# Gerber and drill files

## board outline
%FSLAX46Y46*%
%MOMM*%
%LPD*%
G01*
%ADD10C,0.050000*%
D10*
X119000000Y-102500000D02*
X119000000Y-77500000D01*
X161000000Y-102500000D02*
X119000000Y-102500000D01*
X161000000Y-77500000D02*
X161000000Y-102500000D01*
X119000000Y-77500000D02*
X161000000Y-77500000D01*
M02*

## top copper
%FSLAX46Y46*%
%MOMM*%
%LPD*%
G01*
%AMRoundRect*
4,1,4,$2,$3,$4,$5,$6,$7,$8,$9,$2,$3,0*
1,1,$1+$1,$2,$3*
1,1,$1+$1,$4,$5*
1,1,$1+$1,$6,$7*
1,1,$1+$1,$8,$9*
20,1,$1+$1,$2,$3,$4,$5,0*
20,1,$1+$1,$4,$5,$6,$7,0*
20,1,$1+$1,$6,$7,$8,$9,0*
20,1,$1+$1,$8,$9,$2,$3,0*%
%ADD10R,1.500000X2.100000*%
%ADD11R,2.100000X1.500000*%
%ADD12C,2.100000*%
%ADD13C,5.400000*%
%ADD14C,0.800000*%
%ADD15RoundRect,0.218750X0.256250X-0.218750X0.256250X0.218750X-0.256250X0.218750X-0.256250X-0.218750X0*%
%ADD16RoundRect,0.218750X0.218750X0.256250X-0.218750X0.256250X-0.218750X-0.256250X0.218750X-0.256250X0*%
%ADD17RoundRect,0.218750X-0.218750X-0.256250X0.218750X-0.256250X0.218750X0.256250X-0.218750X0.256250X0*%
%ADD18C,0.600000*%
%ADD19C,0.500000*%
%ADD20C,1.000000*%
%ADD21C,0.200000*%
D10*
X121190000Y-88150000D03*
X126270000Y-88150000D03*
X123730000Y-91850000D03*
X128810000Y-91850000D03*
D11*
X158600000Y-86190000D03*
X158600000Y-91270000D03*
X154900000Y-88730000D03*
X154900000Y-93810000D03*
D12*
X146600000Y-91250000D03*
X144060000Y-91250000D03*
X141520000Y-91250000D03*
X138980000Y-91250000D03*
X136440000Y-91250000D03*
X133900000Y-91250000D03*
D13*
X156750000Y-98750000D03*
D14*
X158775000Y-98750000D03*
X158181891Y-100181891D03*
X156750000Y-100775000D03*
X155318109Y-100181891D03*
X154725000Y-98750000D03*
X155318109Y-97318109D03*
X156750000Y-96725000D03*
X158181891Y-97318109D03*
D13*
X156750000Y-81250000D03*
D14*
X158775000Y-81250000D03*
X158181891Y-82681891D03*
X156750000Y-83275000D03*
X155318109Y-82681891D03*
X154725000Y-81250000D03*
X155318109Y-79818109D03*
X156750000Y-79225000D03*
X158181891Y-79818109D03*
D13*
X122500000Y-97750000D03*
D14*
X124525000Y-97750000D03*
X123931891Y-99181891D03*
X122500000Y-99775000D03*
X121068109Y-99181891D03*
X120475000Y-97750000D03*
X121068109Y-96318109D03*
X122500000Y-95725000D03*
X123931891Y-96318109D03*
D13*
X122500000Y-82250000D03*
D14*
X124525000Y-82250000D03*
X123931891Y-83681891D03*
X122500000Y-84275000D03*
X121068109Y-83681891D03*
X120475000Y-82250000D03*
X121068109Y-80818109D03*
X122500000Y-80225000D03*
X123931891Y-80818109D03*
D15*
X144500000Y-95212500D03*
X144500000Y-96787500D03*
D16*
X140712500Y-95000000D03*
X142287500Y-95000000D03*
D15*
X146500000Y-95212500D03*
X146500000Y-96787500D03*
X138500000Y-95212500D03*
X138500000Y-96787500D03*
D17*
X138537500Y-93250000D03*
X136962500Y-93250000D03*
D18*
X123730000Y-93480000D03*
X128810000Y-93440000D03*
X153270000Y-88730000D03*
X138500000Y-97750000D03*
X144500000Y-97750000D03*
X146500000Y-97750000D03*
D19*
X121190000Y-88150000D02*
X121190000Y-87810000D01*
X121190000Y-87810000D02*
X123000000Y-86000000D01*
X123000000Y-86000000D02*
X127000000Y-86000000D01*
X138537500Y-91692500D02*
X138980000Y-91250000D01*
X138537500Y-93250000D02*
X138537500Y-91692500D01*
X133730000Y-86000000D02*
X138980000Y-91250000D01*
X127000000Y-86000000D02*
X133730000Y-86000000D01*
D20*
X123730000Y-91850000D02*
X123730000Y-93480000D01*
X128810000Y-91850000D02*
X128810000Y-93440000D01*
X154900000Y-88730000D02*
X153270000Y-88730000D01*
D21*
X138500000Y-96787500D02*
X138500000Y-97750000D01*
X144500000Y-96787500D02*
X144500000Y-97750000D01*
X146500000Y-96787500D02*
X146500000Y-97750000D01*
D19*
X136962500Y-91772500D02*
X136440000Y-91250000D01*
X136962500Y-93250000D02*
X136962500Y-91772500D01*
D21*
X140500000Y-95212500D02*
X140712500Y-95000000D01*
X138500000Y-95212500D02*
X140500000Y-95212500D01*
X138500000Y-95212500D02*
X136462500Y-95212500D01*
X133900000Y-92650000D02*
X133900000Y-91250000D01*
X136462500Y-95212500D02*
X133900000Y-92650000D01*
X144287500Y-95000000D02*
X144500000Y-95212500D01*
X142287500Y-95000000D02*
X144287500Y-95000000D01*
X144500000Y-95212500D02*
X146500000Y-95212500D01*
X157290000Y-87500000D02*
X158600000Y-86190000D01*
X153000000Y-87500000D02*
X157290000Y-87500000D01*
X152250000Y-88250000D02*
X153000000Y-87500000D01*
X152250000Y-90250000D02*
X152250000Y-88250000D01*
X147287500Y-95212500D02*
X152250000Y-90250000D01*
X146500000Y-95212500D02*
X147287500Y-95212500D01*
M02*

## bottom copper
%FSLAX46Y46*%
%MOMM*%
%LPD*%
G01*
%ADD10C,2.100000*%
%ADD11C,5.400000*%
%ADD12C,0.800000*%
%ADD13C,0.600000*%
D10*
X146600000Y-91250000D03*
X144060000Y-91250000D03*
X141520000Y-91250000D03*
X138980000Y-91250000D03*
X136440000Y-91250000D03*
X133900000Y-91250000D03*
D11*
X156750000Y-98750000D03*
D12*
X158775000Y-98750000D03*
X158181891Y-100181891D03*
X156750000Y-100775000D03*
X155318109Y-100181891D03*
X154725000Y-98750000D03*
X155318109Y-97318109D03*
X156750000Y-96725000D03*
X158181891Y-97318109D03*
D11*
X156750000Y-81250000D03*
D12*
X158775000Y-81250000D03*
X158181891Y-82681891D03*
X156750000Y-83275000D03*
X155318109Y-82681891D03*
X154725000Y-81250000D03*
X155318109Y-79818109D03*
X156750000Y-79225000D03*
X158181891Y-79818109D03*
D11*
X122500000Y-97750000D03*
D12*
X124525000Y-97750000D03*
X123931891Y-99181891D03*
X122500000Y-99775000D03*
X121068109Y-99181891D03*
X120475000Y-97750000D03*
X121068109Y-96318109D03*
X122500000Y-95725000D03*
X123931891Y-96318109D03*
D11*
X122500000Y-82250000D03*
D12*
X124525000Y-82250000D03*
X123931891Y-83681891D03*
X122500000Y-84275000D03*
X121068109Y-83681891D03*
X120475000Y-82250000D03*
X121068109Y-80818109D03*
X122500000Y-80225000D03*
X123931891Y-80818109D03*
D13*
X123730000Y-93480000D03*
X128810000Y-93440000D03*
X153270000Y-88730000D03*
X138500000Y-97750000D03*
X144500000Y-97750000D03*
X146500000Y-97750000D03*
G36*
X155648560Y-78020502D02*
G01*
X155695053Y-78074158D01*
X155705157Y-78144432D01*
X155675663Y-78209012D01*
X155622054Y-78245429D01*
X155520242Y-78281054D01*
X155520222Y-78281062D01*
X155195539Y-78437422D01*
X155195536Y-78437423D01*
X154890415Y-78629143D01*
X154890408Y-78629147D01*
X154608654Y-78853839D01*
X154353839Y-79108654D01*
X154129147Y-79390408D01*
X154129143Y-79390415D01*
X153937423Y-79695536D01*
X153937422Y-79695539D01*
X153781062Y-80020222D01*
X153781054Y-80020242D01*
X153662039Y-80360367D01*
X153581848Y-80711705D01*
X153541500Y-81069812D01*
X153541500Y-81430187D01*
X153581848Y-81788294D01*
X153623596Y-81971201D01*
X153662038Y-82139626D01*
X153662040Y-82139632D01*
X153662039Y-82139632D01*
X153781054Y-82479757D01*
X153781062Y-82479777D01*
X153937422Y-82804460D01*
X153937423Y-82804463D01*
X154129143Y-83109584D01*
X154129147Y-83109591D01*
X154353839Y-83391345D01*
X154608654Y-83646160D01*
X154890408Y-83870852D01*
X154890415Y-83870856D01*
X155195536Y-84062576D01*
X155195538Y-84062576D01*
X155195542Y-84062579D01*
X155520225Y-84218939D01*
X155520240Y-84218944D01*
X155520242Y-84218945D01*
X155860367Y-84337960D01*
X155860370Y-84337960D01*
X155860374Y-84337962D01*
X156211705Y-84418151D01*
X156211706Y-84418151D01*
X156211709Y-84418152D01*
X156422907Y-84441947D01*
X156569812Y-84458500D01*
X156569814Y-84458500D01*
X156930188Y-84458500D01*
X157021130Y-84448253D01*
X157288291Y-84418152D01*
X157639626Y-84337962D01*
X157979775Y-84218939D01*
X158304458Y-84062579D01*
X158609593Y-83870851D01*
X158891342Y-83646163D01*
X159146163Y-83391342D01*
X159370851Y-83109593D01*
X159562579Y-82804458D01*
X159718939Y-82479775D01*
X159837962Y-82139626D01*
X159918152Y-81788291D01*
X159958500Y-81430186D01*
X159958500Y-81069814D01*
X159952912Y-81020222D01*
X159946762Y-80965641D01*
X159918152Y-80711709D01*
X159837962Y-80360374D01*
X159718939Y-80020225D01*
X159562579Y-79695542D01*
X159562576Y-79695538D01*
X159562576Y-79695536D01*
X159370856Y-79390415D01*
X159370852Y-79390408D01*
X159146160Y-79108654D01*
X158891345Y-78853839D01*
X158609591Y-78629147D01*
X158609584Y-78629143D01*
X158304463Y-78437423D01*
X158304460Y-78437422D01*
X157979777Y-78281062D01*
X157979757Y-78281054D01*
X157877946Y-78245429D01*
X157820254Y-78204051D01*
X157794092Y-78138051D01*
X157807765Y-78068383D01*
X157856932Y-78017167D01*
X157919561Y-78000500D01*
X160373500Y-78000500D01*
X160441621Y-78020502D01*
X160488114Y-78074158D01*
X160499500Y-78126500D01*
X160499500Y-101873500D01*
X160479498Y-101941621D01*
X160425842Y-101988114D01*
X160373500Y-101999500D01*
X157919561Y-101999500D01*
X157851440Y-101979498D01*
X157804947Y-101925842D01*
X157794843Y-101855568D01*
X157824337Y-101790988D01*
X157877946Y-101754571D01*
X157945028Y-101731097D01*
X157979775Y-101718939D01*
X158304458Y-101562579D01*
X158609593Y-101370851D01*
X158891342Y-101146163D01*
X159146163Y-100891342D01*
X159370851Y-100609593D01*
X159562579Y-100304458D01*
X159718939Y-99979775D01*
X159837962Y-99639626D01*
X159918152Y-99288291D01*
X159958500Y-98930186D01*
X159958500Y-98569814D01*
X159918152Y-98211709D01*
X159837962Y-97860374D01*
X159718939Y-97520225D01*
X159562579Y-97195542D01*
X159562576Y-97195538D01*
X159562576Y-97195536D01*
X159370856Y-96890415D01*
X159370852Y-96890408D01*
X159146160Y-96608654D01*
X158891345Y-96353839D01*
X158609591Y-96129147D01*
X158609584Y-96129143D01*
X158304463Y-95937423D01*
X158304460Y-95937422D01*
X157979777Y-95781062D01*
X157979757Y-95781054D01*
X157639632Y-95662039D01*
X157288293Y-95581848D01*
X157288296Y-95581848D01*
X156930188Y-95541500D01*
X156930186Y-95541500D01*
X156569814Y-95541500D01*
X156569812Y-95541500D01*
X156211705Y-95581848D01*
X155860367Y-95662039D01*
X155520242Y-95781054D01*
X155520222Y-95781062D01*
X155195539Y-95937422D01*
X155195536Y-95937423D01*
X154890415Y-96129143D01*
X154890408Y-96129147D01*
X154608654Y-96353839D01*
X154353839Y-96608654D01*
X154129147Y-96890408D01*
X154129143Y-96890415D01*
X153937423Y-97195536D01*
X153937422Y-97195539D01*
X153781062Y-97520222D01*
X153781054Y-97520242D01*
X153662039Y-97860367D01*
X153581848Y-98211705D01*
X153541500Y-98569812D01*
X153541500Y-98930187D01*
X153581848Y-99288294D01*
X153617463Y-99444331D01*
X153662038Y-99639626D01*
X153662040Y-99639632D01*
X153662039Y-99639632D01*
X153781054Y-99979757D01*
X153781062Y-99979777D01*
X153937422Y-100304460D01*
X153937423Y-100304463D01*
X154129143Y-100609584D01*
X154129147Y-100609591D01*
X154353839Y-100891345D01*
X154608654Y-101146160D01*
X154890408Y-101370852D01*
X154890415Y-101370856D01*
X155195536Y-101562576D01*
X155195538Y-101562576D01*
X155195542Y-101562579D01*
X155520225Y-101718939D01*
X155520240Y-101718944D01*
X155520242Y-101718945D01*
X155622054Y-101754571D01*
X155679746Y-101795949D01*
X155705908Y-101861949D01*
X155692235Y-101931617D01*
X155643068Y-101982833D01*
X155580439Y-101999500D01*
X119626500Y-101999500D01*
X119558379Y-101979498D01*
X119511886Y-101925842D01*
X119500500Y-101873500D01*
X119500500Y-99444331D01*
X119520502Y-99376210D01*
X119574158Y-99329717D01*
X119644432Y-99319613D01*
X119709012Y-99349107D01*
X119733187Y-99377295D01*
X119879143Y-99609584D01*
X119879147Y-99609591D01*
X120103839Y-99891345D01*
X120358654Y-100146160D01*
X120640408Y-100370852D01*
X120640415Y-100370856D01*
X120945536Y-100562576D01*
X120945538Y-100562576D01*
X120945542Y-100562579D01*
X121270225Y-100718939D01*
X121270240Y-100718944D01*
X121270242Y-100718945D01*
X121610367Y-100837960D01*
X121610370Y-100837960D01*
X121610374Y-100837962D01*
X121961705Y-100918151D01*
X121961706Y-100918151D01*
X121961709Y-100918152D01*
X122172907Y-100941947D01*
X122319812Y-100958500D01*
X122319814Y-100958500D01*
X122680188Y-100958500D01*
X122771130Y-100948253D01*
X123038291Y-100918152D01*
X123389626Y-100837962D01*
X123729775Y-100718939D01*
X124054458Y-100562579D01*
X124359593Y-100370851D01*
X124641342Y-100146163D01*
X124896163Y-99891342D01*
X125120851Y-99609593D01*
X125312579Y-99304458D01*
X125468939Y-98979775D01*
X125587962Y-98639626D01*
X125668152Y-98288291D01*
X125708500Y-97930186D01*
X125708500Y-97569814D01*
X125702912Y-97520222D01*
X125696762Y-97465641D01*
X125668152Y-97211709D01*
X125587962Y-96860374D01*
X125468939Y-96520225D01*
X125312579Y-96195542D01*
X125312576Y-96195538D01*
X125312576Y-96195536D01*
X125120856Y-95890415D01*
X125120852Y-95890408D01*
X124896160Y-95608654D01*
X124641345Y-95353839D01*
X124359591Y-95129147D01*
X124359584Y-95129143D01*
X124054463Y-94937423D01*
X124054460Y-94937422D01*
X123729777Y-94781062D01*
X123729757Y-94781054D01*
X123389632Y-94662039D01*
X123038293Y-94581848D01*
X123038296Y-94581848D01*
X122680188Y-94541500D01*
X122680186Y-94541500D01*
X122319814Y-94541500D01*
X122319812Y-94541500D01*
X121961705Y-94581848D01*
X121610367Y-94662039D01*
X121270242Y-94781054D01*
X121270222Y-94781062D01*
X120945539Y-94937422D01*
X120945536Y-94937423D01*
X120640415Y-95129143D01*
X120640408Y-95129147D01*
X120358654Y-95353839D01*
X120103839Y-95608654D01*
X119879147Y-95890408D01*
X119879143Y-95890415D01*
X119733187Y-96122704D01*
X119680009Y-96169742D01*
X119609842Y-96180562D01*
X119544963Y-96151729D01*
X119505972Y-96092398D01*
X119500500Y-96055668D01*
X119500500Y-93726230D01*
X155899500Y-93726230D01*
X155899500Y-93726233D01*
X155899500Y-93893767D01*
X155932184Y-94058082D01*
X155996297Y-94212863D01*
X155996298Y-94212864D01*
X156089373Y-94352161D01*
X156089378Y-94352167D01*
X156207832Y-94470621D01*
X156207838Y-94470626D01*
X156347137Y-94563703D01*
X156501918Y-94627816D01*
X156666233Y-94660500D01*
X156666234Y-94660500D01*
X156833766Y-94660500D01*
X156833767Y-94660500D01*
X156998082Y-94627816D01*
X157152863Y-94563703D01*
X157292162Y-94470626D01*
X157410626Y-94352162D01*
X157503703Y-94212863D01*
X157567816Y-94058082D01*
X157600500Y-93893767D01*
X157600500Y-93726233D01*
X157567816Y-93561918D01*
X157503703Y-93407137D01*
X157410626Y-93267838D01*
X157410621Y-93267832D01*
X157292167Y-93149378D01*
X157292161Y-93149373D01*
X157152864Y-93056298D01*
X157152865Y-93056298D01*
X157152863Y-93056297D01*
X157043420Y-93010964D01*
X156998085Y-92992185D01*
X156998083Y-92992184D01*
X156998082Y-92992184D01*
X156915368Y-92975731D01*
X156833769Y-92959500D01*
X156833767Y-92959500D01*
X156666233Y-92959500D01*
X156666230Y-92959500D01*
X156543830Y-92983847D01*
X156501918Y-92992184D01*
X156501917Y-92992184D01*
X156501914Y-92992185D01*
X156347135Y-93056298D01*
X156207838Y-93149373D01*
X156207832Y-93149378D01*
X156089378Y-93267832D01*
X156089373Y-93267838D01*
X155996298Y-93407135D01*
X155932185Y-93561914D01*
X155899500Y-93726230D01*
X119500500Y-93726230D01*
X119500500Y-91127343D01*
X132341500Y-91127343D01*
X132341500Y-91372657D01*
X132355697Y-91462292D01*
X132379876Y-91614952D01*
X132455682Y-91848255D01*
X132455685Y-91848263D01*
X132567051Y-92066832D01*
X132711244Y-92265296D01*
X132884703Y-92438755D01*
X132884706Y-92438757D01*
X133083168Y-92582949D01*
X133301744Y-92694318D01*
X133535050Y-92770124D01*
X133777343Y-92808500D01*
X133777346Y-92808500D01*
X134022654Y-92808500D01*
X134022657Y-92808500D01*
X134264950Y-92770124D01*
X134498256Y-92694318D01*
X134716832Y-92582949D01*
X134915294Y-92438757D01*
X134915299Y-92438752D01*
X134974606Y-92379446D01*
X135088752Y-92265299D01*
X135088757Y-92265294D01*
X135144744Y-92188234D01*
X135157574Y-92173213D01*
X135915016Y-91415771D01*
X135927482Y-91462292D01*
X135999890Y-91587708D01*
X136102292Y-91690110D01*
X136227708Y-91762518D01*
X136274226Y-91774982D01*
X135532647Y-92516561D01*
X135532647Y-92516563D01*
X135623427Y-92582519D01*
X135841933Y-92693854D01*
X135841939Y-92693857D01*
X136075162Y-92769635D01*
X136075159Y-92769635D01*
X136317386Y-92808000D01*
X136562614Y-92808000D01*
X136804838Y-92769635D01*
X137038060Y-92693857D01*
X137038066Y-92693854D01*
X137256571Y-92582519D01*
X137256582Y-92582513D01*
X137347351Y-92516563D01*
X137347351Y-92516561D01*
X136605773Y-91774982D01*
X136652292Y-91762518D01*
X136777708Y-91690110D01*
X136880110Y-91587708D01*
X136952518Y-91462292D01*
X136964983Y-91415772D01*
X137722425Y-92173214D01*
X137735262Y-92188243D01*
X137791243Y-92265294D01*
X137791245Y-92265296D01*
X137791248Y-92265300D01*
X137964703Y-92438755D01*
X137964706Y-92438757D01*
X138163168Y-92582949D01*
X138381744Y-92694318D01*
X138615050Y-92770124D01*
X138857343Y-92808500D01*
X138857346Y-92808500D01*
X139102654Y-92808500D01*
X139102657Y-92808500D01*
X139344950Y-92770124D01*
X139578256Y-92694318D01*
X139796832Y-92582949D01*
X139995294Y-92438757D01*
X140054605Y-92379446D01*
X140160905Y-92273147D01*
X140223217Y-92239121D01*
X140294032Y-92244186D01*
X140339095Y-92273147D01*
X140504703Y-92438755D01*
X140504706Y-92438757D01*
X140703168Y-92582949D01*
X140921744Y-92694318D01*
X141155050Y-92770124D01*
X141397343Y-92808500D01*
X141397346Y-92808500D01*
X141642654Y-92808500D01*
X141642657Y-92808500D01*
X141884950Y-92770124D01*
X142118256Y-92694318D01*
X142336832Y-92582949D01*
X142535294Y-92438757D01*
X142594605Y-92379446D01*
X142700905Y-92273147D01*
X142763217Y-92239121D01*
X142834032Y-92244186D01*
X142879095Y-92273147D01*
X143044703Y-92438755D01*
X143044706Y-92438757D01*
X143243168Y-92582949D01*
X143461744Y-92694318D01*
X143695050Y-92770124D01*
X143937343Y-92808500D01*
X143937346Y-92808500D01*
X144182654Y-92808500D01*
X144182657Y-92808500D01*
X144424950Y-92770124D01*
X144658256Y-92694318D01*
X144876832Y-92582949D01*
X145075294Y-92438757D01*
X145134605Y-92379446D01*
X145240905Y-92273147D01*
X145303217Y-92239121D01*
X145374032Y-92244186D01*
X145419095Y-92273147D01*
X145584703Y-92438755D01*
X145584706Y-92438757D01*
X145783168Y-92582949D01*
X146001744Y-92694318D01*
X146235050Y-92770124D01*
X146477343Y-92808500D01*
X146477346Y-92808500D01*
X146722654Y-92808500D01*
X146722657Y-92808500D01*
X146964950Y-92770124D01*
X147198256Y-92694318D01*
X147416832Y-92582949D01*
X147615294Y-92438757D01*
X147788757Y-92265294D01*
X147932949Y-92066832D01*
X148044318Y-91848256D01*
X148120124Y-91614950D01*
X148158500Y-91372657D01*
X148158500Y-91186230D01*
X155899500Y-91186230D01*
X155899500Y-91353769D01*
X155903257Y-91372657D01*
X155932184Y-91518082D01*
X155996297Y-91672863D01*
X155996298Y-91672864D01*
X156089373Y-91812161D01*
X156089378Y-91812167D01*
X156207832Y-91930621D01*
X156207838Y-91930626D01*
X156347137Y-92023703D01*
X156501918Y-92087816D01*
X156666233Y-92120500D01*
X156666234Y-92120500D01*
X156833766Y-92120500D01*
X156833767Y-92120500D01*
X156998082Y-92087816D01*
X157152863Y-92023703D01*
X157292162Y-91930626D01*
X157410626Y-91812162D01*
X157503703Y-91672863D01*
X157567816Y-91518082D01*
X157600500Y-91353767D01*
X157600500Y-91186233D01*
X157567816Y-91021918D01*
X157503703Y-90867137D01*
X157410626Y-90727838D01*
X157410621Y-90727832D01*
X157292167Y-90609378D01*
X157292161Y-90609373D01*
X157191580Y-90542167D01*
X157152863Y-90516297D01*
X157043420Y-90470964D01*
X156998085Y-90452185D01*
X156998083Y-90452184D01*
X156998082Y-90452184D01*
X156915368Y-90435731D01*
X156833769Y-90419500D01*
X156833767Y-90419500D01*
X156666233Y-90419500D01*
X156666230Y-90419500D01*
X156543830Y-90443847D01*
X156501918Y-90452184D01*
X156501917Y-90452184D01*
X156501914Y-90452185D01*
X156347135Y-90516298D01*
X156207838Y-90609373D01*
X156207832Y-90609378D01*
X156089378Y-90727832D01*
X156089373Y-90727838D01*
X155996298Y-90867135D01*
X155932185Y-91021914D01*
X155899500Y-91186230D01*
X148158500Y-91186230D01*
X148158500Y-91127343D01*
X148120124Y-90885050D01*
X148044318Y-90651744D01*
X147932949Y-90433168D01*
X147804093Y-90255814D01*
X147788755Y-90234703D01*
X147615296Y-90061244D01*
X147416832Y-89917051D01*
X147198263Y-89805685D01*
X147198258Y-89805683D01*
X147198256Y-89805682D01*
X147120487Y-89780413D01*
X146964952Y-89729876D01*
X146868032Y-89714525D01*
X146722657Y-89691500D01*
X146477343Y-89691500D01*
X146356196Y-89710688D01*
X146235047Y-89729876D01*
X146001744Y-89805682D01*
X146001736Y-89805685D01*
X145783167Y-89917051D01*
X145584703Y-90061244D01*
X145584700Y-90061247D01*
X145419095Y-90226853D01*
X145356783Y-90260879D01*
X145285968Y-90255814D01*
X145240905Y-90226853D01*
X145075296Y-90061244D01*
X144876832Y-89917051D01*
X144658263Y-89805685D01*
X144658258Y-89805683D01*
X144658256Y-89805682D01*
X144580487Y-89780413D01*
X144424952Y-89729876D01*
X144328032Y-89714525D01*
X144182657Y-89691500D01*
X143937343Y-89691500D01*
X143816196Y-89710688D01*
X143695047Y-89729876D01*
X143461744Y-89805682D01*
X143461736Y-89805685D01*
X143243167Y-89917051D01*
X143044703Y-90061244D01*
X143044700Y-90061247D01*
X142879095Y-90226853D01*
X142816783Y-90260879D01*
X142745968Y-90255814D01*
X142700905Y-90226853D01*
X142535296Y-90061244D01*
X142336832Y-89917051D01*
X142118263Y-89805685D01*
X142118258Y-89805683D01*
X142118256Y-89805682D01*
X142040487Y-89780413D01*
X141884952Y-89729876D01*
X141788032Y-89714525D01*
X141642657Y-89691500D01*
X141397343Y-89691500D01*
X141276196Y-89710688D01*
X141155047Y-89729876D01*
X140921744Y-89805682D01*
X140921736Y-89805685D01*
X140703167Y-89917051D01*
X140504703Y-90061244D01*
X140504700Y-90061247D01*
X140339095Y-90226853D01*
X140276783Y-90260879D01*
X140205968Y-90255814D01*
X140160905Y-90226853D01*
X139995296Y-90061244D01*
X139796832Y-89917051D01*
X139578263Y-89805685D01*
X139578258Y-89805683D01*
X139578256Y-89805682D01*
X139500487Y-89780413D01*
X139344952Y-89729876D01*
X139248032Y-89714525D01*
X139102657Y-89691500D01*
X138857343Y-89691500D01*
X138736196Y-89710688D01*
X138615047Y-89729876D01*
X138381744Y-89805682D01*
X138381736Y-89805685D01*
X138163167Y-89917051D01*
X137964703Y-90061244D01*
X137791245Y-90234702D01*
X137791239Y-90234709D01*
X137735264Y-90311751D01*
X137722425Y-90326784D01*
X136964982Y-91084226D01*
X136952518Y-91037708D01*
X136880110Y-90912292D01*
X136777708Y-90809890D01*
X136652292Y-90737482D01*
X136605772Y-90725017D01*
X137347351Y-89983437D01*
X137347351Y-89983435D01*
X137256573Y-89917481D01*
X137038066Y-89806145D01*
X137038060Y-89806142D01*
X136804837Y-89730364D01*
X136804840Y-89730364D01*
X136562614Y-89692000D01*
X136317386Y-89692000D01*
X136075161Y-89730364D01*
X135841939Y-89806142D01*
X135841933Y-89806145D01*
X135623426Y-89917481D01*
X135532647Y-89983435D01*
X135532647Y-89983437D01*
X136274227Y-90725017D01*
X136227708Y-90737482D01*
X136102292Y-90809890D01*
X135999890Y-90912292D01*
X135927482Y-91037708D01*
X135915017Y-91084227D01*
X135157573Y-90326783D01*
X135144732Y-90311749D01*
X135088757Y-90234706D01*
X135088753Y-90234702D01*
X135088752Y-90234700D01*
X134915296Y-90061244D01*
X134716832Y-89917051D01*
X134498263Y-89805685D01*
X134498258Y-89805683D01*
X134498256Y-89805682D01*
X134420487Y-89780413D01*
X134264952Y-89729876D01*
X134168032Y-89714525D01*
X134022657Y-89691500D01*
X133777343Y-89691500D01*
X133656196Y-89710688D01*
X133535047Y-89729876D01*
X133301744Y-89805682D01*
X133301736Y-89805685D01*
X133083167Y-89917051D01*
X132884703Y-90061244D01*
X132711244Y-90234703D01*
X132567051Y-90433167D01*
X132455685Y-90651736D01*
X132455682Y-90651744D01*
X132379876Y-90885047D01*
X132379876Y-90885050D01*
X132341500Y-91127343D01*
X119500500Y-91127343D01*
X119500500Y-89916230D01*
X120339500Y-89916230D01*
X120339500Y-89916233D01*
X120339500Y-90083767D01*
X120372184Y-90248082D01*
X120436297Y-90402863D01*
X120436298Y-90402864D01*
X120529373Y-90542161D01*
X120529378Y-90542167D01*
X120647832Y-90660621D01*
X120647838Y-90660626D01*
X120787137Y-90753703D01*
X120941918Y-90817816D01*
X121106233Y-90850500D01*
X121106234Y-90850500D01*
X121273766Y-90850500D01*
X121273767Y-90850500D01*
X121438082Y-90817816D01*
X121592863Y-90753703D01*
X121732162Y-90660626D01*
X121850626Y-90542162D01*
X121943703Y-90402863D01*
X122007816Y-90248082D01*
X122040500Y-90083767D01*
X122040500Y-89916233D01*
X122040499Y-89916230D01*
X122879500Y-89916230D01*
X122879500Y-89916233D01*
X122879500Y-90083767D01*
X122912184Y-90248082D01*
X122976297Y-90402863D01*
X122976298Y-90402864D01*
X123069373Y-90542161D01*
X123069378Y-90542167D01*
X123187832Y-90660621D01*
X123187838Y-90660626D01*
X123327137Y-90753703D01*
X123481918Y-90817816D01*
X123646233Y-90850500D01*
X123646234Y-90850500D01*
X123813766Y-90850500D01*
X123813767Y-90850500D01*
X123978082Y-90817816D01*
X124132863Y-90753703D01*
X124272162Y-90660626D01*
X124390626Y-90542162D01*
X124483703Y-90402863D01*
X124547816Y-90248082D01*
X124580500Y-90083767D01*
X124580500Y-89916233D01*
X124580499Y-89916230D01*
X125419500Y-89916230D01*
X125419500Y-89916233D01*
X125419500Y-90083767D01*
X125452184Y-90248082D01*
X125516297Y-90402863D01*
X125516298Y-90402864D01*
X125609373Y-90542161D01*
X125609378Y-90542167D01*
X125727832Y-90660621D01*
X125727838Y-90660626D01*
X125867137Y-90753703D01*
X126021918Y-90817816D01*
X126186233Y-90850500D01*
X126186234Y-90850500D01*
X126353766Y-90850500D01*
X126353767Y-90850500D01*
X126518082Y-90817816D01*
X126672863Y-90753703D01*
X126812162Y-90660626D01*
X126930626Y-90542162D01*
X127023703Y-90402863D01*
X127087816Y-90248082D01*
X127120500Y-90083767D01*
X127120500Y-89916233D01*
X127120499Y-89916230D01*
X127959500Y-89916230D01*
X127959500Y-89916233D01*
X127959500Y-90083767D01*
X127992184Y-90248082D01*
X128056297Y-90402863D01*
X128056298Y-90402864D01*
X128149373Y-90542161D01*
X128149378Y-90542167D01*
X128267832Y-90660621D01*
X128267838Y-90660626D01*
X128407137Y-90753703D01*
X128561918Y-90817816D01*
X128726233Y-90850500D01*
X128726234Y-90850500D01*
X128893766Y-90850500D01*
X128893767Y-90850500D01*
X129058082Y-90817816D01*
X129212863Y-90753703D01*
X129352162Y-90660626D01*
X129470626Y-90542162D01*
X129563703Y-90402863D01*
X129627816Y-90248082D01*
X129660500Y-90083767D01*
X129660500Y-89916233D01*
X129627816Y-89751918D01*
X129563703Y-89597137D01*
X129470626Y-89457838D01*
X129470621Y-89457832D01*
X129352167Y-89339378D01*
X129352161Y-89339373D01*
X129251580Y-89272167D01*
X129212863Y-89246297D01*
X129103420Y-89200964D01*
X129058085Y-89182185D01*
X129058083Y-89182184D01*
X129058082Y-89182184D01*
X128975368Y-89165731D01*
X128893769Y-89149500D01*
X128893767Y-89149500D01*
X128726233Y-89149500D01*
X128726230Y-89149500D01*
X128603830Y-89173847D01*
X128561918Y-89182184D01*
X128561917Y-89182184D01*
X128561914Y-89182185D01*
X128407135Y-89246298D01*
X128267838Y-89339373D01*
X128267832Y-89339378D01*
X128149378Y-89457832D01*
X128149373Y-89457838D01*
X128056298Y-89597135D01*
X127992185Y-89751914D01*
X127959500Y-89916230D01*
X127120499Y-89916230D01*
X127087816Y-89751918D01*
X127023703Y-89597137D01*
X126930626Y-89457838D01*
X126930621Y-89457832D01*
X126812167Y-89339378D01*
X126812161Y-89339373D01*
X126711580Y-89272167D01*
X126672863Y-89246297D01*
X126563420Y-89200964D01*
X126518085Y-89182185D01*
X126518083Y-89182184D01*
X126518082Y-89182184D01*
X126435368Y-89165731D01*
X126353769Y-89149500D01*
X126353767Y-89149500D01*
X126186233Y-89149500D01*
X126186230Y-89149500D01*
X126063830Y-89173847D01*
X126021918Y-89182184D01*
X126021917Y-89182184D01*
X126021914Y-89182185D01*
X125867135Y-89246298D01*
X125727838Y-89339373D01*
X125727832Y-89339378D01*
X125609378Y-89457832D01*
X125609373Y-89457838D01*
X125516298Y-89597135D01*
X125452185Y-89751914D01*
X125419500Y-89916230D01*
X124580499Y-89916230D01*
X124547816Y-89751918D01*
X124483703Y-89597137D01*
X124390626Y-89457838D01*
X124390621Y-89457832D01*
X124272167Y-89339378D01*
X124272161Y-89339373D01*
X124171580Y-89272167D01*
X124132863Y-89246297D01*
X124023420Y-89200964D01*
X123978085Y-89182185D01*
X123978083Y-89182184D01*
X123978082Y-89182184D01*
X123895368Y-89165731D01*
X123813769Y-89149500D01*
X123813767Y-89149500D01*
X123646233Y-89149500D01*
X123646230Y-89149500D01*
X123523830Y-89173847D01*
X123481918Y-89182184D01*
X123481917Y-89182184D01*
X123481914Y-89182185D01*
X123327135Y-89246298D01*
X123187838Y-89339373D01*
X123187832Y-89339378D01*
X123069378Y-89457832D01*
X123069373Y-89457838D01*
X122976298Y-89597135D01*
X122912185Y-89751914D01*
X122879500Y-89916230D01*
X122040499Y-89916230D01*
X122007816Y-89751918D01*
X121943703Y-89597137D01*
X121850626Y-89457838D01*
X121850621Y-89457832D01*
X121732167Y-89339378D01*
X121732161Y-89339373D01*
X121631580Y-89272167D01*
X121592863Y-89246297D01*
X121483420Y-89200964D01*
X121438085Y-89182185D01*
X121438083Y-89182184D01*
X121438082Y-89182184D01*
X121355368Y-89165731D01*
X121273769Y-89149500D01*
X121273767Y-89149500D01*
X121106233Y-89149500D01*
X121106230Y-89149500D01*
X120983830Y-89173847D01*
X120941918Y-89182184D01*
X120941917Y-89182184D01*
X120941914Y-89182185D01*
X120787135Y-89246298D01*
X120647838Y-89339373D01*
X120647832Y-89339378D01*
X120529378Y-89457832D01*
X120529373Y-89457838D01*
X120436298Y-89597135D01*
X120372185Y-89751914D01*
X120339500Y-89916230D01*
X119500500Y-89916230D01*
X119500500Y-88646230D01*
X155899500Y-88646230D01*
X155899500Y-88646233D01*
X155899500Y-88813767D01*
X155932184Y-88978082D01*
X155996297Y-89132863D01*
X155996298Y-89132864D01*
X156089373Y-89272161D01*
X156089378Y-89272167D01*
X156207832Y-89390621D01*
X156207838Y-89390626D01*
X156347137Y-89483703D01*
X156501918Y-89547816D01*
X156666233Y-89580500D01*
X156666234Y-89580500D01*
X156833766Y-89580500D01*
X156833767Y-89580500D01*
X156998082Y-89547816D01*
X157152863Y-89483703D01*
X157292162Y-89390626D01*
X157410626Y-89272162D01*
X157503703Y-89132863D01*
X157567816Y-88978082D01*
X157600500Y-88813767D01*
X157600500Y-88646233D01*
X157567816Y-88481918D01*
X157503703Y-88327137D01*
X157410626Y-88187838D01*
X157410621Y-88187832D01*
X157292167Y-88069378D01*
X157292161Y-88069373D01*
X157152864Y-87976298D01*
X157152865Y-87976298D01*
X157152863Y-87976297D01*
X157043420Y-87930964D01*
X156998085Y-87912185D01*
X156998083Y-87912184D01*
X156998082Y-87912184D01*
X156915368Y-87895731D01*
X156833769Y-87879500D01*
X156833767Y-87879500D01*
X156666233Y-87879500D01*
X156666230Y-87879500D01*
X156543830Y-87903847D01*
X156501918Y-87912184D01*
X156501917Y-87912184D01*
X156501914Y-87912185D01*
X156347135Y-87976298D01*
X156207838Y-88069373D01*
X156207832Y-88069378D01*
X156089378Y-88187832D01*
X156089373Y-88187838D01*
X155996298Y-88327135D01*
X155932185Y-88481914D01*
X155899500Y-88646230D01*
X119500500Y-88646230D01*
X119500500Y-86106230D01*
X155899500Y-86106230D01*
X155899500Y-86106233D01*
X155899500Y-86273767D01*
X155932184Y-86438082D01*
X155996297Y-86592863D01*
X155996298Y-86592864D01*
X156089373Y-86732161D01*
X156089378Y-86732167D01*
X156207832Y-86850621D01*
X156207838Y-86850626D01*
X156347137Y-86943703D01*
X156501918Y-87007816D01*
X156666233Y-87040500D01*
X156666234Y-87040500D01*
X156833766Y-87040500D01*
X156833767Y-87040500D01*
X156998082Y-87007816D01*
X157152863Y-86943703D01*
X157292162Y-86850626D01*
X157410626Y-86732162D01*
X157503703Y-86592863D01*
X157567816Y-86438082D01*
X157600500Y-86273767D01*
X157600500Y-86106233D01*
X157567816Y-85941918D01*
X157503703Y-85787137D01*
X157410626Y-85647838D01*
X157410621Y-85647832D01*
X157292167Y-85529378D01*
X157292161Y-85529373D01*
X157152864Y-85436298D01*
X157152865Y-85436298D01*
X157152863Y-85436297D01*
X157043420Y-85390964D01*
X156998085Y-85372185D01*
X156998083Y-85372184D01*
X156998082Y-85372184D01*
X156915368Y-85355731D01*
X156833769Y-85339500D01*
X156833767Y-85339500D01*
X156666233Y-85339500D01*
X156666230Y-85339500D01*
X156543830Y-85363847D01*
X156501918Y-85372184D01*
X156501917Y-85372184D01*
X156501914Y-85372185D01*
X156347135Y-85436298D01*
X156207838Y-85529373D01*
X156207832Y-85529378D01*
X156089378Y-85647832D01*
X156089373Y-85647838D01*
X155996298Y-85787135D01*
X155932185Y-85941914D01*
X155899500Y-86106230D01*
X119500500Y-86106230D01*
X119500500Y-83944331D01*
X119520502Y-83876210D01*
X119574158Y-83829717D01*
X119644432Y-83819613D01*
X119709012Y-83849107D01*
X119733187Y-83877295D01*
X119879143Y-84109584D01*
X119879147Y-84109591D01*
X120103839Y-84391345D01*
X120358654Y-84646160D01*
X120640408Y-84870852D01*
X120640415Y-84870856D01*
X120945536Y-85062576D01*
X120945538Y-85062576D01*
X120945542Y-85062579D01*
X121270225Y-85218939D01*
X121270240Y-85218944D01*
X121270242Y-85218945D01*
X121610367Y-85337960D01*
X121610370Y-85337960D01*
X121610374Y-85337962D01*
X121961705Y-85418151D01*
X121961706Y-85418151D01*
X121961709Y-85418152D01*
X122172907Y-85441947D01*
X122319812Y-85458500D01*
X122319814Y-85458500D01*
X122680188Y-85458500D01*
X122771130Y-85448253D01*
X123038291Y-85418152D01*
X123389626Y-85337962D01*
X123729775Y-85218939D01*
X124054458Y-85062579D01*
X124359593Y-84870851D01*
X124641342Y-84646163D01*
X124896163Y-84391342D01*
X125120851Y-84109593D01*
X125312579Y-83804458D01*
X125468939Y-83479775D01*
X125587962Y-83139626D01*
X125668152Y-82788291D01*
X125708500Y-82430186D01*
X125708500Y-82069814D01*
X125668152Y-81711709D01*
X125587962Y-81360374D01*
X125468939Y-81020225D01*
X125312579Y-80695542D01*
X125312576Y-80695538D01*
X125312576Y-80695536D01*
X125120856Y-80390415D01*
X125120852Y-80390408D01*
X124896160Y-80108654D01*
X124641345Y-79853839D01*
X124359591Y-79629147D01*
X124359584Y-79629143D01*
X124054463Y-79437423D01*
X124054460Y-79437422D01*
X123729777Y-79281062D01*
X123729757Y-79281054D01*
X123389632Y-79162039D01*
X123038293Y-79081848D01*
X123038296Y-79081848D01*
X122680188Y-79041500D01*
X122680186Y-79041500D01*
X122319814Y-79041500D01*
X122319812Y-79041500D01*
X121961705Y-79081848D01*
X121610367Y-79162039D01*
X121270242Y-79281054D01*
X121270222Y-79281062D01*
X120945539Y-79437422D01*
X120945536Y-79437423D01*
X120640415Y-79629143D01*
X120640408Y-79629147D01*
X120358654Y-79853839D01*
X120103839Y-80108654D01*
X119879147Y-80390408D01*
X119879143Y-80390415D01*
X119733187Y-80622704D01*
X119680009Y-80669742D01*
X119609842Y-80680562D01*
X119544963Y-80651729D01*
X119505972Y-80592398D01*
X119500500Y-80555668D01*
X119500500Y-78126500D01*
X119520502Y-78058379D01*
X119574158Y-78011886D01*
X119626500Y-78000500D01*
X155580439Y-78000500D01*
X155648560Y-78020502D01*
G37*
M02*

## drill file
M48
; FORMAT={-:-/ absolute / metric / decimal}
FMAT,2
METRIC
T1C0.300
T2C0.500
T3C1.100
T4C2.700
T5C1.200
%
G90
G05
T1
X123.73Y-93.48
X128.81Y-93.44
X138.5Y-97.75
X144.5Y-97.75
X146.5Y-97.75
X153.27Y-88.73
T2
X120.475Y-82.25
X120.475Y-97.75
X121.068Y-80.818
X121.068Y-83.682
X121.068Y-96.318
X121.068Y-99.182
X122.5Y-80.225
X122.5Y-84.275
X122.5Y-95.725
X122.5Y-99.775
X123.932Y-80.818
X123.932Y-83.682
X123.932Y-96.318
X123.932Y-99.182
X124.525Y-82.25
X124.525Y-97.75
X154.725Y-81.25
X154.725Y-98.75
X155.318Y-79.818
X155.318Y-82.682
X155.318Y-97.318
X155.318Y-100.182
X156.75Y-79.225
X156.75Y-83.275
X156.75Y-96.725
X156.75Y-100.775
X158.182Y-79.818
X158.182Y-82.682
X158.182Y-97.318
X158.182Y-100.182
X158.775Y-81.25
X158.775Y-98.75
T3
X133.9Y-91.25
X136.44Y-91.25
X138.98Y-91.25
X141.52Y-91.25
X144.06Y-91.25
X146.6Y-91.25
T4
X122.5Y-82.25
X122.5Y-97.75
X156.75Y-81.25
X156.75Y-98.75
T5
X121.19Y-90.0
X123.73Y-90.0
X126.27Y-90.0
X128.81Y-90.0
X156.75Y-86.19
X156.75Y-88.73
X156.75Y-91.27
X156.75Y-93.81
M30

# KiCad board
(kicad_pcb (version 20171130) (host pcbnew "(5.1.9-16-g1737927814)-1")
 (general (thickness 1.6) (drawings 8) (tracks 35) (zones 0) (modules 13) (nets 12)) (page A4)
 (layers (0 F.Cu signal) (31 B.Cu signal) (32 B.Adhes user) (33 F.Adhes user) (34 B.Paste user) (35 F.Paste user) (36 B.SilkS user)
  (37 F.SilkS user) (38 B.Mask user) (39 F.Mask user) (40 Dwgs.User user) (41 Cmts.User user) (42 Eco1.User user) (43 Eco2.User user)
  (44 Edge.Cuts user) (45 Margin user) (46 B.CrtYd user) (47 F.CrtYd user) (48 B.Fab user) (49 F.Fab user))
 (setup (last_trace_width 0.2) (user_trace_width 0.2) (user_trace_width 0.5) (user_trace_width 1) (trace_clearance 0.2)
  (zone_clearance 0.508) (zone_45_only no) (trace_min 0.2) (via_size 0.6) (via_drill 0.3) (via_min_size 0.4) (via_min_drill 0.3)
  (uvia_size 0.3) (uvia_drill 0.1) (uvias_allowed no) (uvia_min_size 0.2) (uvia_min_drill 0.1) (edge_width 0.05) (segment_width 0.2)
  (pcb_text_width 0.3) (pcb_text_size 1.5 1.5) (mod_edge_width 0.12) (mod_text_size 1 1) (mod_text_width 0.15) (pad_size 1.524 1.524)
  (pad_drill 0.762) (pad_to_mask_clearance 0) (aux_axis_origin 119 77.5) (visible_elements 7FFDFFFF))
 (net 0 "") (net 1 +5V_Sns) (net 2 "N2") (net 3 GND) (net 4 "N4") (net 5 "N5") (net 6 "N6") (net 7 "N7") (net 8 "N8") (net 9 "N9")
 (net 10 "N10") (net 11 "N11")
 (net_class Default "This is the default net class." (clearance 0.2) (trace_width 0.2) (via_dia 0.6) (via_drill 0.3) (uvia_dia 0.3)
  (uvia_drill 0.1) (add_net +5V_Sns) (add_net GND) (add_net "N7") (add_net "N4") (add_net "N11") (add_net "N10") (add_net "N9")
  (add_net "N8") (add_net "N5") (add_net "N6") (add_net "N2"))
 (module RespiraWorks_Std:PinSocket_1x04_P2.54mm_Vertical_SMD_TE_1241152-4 (layer F.Cu) (at 125 90 90)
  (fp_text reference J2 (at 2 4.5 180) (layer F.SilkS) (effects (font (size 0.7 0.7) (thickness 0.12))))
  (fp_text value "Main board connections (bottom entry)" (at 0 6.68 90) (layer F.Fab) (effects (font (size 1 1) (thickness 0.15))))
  (pad "" np_thru_hole circle (at 0 1.27 90) (size 1.2 1.2) (drill 1.2) (layers *.Cu *.Mask))
  (pad "" np_thru_hole circle (at 0 -1.27 90) (size 1.2 1.2) (drill 1.2) (layers *.Cu *.Mask))
  (pad "" np_thru_hole circle (at 0 -3.81 90) (size 1.2 1.2) (drill 1.2) (layers *.Cu *.Mask))
  (pad 1 smd rect (at 1.85 -3.81 90) (size 2.1 1.5) (layers F.Cu F.Paste F.Mask) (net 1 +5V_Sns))
  (pad 3 smd rect (at 1.85 1.27 90) (size 2.1 1.5) (layers F.Cu F.Paste F.Mask) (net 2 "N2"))
  (pad 2 smd rect (at -1.85 -1.27 90) (size 2.1 1.5) (layers F.Cu F.Paste F.Mask) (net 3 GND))
  (pad 4 smd rect (at -1.85 3.81 90) (size 2.1 1.5) (layers F.Cu F.Paste F.Mask) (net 3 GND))
  (pad "" np_thru_hole circle (at 0 3.81 90) (size 1.2 1.2) (drill 1.2) (layers *.Cu *.Mask)))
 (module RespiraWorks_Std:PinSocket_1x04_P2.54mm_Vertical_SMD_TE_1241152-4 (layer F.Cu) (at 156.75 90)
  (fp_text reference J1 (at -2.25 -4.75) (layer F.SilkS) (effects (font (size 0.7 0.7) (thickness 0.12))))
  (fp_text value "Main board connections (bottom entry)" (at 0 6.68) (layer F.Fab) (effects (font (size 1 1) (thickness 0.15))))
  (pad "" np_thru_hole circle (at 0 1.27) (size 1.2 1.2) (drill 1.2) (layers *.Cu *.Mask))
  (pad "" np_thru_hole circle (at 0 -1.27) (size 1.2 1.2) (drill 1.2) (layers *.Cu *.Mask))
  (pad "" np_thru_hole circle (at 0 -3.81) (size 1.2 1.2) (drill 1.2) (layers *.Cu *.Mask))
  (pad 1 smd rect (at 1.85 -3.81) (size 2.1 1.5) (layers F.Cu F.Paste F.Mask) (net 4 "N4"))
  (pad 3 smd rect (at 1.85 1.27) (size 2.1 1.5) (layers F.Cu F.Paste F.Mask) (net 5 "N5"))
  (pad 2 smd rect (at -1.85 -1.27) (size 2.1 1.5) (layers F.Cu F.Paste F.Mask) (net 3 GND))
  (pad 4 smd rect (at -1.85 3.81) (size 2.1 1.5) (layers F.Cu F.Paste F.Mask) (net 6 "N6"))
  (pad "" np_thru_hole circle (at 0 3.81) (size 1.2 1.2) (drill 1.2) (layers *.Cu *.Mask)))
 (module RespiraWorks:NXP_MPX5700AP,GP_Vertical (layer F.Cu) (at 140.25 91.25)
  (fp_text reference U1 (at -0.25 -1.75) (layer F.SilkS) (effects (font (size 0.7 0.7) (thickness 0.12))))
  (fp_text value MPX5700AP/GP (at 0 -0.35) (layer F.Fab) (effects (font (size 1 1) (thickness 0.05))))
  (pad 6 thru_hole circle (at 6.35 0) (size 2.1 2.1) (drill 1.1) (layers *.Cu *.Mask))
  (pad 5 thru_hole circle (at 3.81 0) (size 2.1 2.1) (drill 1.1) (layers *.Cu *.Mask))
  (pad 4 thru_hole circle (at 1.27 0) (size 2.1 2.1) (drill 1.1) (layers *.Cu *.Mask))
  (pad 3 thru_hole circle (at -1.27 0) (size 2.1 2.1) (drill 1.1) (layers *.Cu *.Mask) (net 1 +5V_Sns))
  (pad 2 thru_hole circle (at -3.81 0) (size 2.1 2.1) (drill 1.1) (layers *.Cu *.Mask) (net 3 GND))
  (pad 1 thru_hole circle (at -6.35 0) (size 2.1 2.1) (drill 1.1) (layers *.Cu *.Mask) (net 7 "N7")))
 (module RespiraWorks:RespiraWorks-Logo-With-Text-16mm (layer B.Cu) (at 139.5 89.75 180)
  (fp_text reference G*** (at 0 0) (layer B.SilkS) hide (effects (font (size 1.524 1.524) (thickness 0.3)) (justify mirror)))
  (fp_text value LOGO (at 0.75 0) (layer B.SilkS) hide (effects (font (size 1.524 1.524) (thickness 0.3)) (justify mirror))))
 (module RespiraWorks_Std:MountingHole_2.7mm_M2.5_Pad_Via (layer F.Cu) (at 156.75 98.75)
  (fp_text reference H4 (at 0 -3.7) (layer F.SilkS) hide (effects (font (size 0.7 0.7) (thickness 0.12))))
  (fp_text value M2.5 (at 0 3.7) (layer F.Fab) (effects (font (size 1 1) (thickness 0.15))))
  (pad 1 thru_hole circle (at 0 0) (size 5.4 5.4) (drill 2.7) (layers *.Cu *.Mask) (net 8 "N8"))
  (pad 1 thru_hole circle (at 2.025 0) (size 0.8 0.8) (drill 0.5) (layers *.Cu *.Mask) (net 8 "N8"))
  (pad 1 thru_hole circle (at 1.431891 1.431891) (size 0.8 0.8) (drill 0.5) (layers *.Cu *.Mask) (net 8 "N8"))
  (pad 1 thru_hole circle (at 0 2.025) (size 0.8 0.8) (drill 0.5) (layers *.Cu *.Mask) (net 8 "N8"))
  (pad 1 thru_hole circle (at -1.431891 1.431891) (size 0.8 0.8) (drill 0.5) (layers *.Cu *.Mask) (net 8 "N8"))
  (pad 1 thru_hole circle (at -2.025 0) (size 0.8 0.8) (drill 0.5) (layers *.Cu *.Mask) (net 8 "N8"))
  (pad 1 thru_hole circle (at -1.431891 -1.431891) (size 0.8 0.8) (drill 0.5) (layers *.Cu *.Mask) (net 8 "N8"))
  (pad 1 thru_hole circle (at 0 -2.025) (size 0.8 0.8) (drill 0.5) (layers *.Cu *.Mask) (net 8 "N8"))
  (pad 1 thru_hole circle (at 1.431891 -1.431891) (size 0.8 0.8) (drill 0.5) (layers *.Cu *.Mask) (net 8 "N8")))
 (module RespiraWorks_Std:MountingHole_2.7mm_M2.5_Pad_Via (layer F.Cu) (at 156.75 81.25)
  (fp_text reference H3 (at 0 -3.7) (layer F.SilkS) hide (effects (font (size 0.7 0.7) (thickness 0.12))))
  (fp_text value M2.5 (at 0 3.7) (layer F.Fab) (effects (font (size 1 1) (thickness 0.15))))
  (pad 1 thru_hole circle (at 0 0) (size 5.4 5.4) (drill 2.7) (layers *.Cu *.Mask) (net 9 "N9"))
  (pad 1 thru_hole circle (at 2.025 0) (size 0.8 0.8) (drill 0.5) (layers *.Cu *.Mask) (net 9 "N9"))
  (pad 1 thru_hole circle (at 1.431891 1.431891) (size 0.8 0.8) (drill 0.5) (layers *.Cu *.Mask) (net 9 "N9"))
  (pad 1 thru_hole circle (at 0 2.025) (size 0.8 0.8) (drill 0.5) (layers *.Cu *.Mask) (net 9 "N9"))
  (pad 1 thru_hole circle (at -1.431891 1.431891) (size 0.8 0.8) (drill 0.5) (layers *.Cu *.Mask) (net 9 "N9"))
  (pad 1 thru_hole circle (at -2.025 0) (size 0.8 0.8) (drill 0.5) (layers *.Cu *.Mask) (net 9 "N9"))
  (pad 1 thru_hole circle (at -1.431891 -1.431891) (size 0.8 0.8) (drill 0.5) (layers *.Cu *.Mask) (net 9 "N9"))
  (pad 1 thru_hole circle (at 0 -2.025) (size 0.8 0.8) (drill 0.5) (layers *.Cu *.Mask) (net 9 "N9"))
  (pad 1 thru_hole circle (at 1.431891 -1.431891) (size 0.8 0.8) (drill 0.5) (layers *.Cu *.Mask) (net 9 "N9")))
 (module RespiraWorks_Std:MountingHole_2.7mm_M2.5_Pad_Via (layer F.Cu) (at 122.5 97.75)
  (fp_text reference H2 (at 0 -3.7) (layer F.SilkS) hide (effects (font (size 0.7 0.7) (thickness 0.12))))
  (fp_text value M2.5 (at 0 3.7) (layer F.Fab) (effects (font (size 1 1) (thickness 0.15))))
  (pad 1 thru_hole circle (at 0 0) (size 5.4 5.4) (drill 2.7) (layers *.Cu *.Mask) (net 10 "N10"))
  (pad 1 thru_hole circle (at 2.025 0) (size 0.8 0.8) (drill 0.5) (layers *.Cu *.Mask) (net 10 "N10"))
  (pad 1 thru_hole circle (at 1.431891 1.431891) (size 0.8 0.8) (drill 0.5) (layers *.Cu *.Mask) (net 10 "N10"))
  (pad 1 thru_hole circle (at 0 2.025) (size 0.8 0.8) (drill 0.5) (layers *.Cu *.Mask) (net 10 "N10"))
  (pad 1 thru_hole circle (at -1.431891 1.431891) (size 0.8 0.8) (drill 0.5) (layers *.Cu *.Mask) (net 10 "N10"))
  (pad 1 thru_hole circle (at -2.025 0) (size 0.8 0.8) (drill 0.5) (layers *.Cu *.Mask) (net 10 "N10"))
  (pad 1 thru_hole circle (at -1.431891 -1.431891) (size 0.8 0.8) (drill 0.5) (layers *.Cu *.Mask) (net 10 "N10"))
  (pad 1 thru_hole circle (at 0 -2.025) (size 0.8 0.8) (drill 0.5) (layers *.Cu *.Mask) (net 10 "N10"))
  (pad 1 thru_hole circle (at 1.431891 -1.431891) (size 0.8 0.8) (drill 0.5) (layers *.Cu *.Mask) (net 10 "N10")))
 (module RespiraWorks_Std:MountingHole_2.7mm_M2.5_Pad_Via (layer F.Cu) (at 122.5 82.25)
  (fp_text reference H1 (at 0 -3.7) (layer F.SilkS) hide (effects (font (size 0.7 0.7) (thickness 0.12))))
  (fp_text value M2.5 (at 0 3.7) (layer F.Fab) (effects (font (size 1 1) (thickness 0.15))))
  (pad 1 thru_hole circle (at 0 0) (size 5.4 5.4) (drill 2.7) (layers *.Cu *.Mask) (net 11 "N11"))
  (pad 1 thru_hole circle (at 2.025 0) (size 0.8 0.8) (drill 0.5) (layers *.Cu *.Mask) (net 11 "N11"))
  (pad 1 thru_hole circle (at 1.431891 1.431891) (size 0.8 0.8) (drill 0.5) (layers *.Cu *.Mask) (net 11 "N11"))
  (pad 1 thru_hole circle (at 0 2.025) (size 0.8 0.8) (drill 0.5) (layers *.Cu *.Mask) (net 11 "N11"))
  (pad 1 thru_hole circle (at -1.431891 1.431891) (size 0.8 0.8) (drill 0.5) (layers *.Cu *.Mask) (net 11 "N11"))
  (pad 1 thru_hole circle (at -2.025 0) (size 0.8 0.8) (drill 0.5) (layers *.Cu *.Mask) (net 11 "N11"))
  (pad 1 thru_hole circle (at -1.431891 -1.431891) (size 0.8 0.8) (drill 0.5) (layers *.Cu *.Mask) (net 11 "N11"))
  (pad 1 thru_hole circle (at 0 -2.025) (size 0.8 0.8) (drill 0.5) (layers *.Cu *.Mask) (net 11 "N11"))
  (pad 1 thru_hole circle (at 1.431891 -1.431891) (size 0.8 0.8) (drill 0.5) (layers *.Cu *.Mask) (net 11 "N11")))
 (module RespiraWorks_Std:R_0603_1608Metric (layer F.Cu) (at 144.5 96 90)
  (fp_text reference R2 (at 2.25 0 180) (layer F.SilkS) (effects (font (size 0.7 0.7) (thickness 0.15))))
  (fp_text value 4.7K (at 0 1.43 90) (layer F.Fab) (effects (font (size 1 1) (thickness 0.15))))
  (pad 2 smd roundrect (at 0.7875 0 90) (size 0.875 0.95) (layers F.Cu F.Paste F.Mask) (roundrect_rratio 0.25) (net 4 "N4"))
  (pad 1 smd roundrect (at -0.7875 0 90) (size 0.875 0.95) (layers F.Cu F.Paste F.Mask) (roundrect_rratio 0.25) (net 3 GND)))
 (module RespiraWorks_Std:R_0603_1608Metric (layer F.Cu) (at 141.5 95 180)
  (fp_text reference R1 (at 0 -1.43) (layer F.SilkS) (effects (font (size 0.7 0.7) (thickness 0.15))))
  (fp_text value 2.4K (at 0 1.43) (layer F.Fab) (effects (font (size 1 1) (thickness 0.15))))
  (pad 2 smd roundrect (at 0.7875 0 180) (size 0.875 0.95) (layers F.Cu F.Paste F.Mask) (roundrect_rratio 0.25) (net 7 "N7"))
  (pad 1 smd roundrect (at -0.7875 0 180) (size 0.875 0.95) (layers F.Cu F.Paste F.Mask) (roundrect_rratio 0.25) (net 4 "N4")))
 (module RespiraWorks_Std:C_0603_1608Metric (layer F.Cu) (at 146.5 96 90)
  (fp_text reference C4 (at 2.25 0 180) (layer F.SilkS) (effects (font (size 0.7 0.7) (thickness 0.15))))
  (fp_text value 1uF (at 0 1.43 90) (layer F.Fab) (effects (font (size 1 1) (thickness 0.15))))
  (pad 2 smd roundrect (at 0.7875 0 90) (size 0.875 0.95) (layers F.Cu F.Paste F.Mask) (roundrect_rratio 0.25) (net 4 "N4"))
  (pad 1 smd roundrect (at -0.7875 0 90) (size 0.875 0.95) (layers F.Cu F.Paste F.Mask) (roundrect_rratio 0.25) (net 3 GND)))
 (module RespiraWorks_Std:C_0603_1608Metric (layer F.Cu) (at 138.5 96 90)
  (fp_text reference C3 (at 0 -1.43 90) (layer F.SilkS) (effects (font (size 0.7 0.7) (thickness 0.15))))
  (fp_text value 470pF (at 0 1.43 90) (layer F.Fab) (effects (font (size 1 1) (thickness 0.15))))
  (pad 2 smd roundrect (at 0.7875 0 90) (size 0.875 0.95) (layers F.Cu F.Paste F.Mask) (roundrect_rratio 0.25) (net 7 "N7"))
  (pad 1 smd roundrect (at -0.7875 0 90) (size 0.875 0.95) (layers F.Cu F.Paste F.Mask) (roundrect_rratio 0.25) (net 3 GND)))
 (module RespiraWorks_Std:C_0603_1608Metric (layer F.Cu) (at 137.75 93.25)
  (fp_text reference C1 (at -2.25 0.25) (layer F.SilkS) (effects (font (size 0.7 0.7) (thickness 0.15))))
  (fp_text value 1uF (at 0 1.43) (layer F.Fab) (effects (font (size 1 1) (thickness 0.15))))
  (pad 2 smd roundrect (at 0.7875 0) (size 0.875 0.95) (layers F.Cu F.Paste F.Mask) (roundrect_rratio 0.25) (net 1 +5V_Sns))
  (pad 1 smd roundrect (at -0.7875 0) (size 0.875 0.95) (layers F.Cu F.Paste F.Mask) (roundrect_rratio 0.25) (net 3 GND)))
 (gr_line (start 119 102.5) (end 119 77.5) (layer Edge.Cuts) (width 0.05))
 (gr_line (start 161 102.5) (end 119 102.5) (layer Edge.Cuts) (width 0.05))
 (gr_line (start 161 77.5) (end 161 102.5) (layer Edge.Cuts) (width 0.05))
 (gr_line (start 119 77.5) (end 161 77.5) (layer Edge.Cuts) (width 0.05))
 (segment (start 121.19 88.15) (end 121.19 87.81) (width 0.5) (layer F.Cu) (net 1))
 (segment (start 121.19 87.81) (end 123 86) (width 0.5) (layer F.Cu) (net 1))
 (segment (start 123 86) (end 127 86) (width 0.5) (layer F.Cu) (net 1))
 (segment (start 138.5375 91.6925) (end 138.98 91.25) (width 0.5) (layer F.Cu) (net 1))
 (segment (start 138.5375 93.25) (end 138.5375 91.6925) (width 0.5) (layer F.Cu) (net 1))
 (segment (start 133.73 86) (end 138.98 91.25) (width 0.5) (layer F.Cu) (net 1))
 (segment (start 127 86) (end 133.73 86) (width 0.5) (layer F.Cu) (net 1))
 (segment (start 123.73 91.85) (end 123.73 93.48) (width 1) (layer F.Cu) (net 3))
 (via (at 123.73 93.48) (size 0.6) (drill 0.3) (layers F.Cu B.Cu) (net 3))
 (segment (start 128.81 91.85) (end 128.81 93.44) (width 1) (layer F.Cu) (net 3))
 (via (at 128.81 93.44) (size 0.6) (drill 0.3) (layers F.Cu B.Cu) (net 3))
 (segment (start 154.9 88.73) (end 153.27 88.73) (width 1) (layer F.Cu) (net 3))
 (via (at 153.27 88.73) (size 0.6) (drill 0.3) (layers F.Cu B.Cu) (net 3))
 (segment (start 138.5 96.7875) (end 138.5 97.75) (width 0.2) (layer F.Cu) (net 3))
 (via (at 138.5 97.75) (size 0.6) (drill 0.3) (layers F.Cu B.Cu) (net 3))
 (segment (start 144.5 96.7875) (end 144.5 97.75) (width 0.2) (layer F.Cu) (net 3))
 (via (at 144.5 97.75) (size 0.6) (drill 0.3) (layers F.Cu B.Cu) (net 3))
 (segment (start 146.5 96.7875) (end 146.5 97.75) (width 0.2) (layer F.Cu) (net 3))
 (via (at 146.5 97.75) (size 0.6) (drill 0.3) (layers F.Cu B.Cu) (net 3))
 (segment (start 136.9625 91.7725) (end 136.44 91.25) (width 0.5) (layer F.Cu) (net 3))
 (segment (start 136.9625 93.25) (end 136.9625 91.7725) (width 0.5) (layer F.Cu) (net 3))
 (segment (start 140.5 95.2125) (end 140.7125 95) (width 0.2) (layer F.Cu) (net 7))
 (segment (start 138.5 95.2125) (end 140.5 95.2125) (width 0.2) (layer F.Cu) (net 7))
 (segment (start 138.5 95.2125) (end 136.4625 95.2125) (width 0.2) (layer F.Cu) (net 7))
 (segment (start 133.9 92.65) (end 133.9 91.25) (width 0.2) (layer F.Cu) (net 7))
 (segment (start 136.4625 95.2125) (end 133.9 92.65) (width 0.2) (layer F.Cu) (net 7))
 (segment (start 144.2875 95) (end 144.5 95.2125) (width 0.2) (layer F.Cu) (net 4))
 (segment (start 142.2875 95) (end 144.2875 95) (width 0.2) (layer F.Cu) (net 4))
 (segment (start 144.5 95.2125) (end 146.5 95.2125) (width 0.2) (layer F.Cu) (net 4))
 (segment (start 157.29 87.5) (end 158.6 86.19) (width 0.2) (layer F.Cu) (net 4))
 (segment (start 153 87.5) (end 157.29 87.5) (width 0.2) (layer F.Cu) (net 4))
 (segment (start 152.25 88.25) (end 153 87.5) (width 0.2) (layer F.Cu) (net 4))
 (segment (start 152.25 90.25) (end 152.25 88.25) (width 0.2) (layer F.Cu) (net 4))
 (segment (start 147.2875 95.2125) (end 152.25 90.25) (width 0.2) (layer F.Cu) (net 4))
 (segment (start 146.5 95.2125) (end 147.2875 95.2125) (width 0.2) (layer F.Cu) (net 4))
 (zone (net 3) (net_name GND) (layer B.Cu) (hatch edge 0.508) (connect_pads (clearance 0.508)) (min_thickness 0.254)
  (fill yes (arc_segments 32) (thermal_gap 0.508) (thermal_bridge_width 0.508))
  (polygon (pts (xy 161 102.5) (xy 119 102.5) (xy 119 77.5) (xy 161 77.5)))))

